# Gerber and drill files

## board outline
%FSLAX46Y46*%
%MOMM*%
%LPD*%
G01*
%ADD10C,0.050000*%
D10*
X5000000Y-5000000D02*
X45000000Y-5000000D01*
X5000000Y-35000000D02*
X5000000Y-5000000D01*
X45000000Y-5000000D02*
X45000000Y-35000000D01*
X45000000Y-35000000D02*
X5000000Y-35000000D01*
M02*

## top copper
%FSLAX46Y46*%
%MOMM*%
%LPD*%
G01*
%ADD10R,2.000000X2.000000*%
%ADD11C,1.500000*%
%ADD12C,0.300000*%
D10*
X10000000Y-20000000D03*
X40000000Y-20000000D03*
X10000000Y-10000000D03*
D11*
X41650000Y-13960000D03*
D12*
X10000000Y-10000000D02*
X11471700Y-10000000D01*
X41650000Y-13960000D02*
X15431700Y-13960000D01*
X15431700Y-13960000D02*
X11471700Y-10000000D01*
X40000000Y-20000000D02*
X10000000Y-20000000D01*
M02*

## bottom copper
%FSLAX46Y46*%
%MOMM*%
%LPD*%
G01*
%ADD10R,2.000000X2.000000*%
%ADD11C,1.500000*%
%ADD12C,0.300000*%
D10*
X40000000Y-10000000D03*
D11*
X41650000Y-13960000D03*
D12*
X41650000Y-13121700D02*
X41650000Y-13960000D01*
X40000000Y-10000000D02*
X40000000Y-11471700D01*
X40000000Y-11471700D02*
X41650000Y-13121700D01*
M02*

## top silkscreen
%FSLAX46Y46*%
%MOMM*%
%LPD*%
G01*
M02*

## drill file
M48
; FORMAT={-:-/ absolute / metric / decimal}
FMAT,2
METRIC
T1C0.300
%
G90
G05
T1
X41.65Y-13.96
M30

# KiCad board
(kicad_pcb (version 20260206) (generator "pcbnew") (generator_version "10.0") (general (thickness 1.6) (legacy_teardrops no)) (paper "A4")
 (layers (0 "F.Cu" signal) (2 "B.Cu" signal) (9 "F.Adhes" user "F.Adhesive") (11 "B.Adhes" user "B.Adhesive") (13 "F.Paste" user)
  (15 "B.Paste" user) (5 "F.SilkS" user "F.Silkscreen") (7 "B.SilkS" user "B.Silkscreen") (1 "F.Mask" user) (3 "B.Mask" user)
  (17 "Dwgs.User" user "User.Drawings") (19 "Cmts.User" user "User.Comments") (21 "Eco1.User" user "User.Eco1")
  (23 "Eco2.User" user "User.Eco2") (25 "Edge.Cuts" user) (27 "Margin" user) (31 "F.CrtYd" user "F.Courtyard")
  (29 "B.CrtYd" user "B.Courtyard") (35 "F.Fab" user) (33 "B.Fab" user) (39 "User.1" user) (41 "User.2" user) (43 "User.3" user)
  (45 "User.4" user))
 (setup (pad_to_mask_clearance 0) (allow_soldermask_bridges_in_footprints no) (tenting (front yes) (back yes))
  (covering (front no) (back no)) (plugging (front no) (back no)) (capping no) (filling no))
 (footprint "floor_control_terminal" (layer "F.Cu") (at 10 20)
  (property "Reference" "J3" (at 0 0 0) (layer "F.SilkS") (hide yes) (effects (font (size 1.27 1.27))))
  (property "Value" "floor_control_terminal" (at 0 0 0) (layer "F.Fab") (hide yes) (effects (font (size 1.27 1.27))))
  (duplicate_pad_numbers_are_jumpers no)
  (pad "1" smd rect (at 0 0) (size 2 2) (layers "F.Cu" "F.Mask" "F.Paste") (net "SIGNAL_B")))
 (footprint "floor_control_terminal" (layer "F.Cu") (at 40 20)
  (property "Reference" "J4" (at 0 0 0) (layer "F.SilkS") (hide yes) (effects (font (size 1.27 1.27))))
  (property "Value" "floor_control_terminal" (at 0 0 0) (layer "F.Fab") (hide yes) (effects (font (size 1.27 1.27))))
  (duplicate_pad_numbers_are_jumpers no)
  (pad "1" smd rect (at 0 0) (size 2 2) (layers "F.Cu" "F.Mask" "F.Paste") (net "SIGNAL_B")))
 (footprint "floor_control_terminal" (layer "F.Cu") (at 10 10)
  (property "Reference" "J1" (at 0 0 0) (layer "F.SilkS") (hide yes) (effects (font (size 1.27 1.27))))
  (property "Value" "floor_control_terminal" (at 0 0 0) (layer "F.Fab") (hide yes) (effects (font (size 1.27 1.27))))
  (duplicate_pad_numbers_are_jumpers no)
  (pad "1" smd rect (at 0 0) (size 2 2) (layers "F.Cu" "F.Mask" "F.Paste") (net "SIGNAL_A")))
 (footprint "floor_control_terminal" (layer "B.Cu") (at 40 10)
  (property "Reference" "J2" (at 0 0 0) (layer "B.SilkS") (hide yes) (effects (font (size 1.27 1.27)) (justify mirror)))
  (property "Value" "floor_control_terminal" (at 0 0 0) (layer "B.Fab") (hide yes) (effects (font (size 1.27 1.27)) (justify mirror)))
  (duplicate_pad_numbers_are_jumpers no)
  (pad "1" smd rect (at 0 0) (size 2 2) (layers "B.Cu" "B.Mask" "B.Paste") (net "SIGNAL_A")))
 (gr_line (start 5 5) (end 45 5) (stroke (width 0.05) (type default)) (layer "Edge.Cuts"))
 (gr_line (start 5 35) (end 5 5) (stroke (width 0.05) (type default)) (layer "Edge.Cuts"))
 (gr_line (start 45 5) (end 45 35) (stroke (width 0.05) (type default)) (layer "Edge.Cuts"))
 (gr_line (start 45 35) (end 5 35) (stroke (width 0.05) (type default)) (layer "Edge.Cuts"))
 (segment (start 10 10) (end 11.4717 10) (width 0.3) (layer "F.Cu") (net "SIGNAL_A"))
 (segment (start 41.65 13.96) (end 15.4317 13.96) (width 0.3) (layer "F.Cu") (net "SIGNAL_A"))
 (segment (start 15.4317 13.96) (end 11.4717 10) (width 0.3) (layer "F.Cu") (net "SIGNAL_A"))
 (via (at 41.65 13.96) (size 1.5) (drill 0.3) (layers "F.Cu" "B.Cu") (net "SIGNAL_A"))
 (segment (start 41.65 13.1217) (end 41.65 13.96) (width 0.3) (layer "B.Cu") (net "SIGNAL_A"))
 (segment (start 40 10) (end 40 11.4717) (width 0.3) (layer "B.Cu") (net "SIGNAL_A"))
 (segment (start 40 11.4717) (end 41.65 13.1217) (width 0.3) (layer "B.Cu") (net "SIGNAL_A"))
 (segment (start 40 20) (end 10 20) (width 0.3) (layer "F.Cu") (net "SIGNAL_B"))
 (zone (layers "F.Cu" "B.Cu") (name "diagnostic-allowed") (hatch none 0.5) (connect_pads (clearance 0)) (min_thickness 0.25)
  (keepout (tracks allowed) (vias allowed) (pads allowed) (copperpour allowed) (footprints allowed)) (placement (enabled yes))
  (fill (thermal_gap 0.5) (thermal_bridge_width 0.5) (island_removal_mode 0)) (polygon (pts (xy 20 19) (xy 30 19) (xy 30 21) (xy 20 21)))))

